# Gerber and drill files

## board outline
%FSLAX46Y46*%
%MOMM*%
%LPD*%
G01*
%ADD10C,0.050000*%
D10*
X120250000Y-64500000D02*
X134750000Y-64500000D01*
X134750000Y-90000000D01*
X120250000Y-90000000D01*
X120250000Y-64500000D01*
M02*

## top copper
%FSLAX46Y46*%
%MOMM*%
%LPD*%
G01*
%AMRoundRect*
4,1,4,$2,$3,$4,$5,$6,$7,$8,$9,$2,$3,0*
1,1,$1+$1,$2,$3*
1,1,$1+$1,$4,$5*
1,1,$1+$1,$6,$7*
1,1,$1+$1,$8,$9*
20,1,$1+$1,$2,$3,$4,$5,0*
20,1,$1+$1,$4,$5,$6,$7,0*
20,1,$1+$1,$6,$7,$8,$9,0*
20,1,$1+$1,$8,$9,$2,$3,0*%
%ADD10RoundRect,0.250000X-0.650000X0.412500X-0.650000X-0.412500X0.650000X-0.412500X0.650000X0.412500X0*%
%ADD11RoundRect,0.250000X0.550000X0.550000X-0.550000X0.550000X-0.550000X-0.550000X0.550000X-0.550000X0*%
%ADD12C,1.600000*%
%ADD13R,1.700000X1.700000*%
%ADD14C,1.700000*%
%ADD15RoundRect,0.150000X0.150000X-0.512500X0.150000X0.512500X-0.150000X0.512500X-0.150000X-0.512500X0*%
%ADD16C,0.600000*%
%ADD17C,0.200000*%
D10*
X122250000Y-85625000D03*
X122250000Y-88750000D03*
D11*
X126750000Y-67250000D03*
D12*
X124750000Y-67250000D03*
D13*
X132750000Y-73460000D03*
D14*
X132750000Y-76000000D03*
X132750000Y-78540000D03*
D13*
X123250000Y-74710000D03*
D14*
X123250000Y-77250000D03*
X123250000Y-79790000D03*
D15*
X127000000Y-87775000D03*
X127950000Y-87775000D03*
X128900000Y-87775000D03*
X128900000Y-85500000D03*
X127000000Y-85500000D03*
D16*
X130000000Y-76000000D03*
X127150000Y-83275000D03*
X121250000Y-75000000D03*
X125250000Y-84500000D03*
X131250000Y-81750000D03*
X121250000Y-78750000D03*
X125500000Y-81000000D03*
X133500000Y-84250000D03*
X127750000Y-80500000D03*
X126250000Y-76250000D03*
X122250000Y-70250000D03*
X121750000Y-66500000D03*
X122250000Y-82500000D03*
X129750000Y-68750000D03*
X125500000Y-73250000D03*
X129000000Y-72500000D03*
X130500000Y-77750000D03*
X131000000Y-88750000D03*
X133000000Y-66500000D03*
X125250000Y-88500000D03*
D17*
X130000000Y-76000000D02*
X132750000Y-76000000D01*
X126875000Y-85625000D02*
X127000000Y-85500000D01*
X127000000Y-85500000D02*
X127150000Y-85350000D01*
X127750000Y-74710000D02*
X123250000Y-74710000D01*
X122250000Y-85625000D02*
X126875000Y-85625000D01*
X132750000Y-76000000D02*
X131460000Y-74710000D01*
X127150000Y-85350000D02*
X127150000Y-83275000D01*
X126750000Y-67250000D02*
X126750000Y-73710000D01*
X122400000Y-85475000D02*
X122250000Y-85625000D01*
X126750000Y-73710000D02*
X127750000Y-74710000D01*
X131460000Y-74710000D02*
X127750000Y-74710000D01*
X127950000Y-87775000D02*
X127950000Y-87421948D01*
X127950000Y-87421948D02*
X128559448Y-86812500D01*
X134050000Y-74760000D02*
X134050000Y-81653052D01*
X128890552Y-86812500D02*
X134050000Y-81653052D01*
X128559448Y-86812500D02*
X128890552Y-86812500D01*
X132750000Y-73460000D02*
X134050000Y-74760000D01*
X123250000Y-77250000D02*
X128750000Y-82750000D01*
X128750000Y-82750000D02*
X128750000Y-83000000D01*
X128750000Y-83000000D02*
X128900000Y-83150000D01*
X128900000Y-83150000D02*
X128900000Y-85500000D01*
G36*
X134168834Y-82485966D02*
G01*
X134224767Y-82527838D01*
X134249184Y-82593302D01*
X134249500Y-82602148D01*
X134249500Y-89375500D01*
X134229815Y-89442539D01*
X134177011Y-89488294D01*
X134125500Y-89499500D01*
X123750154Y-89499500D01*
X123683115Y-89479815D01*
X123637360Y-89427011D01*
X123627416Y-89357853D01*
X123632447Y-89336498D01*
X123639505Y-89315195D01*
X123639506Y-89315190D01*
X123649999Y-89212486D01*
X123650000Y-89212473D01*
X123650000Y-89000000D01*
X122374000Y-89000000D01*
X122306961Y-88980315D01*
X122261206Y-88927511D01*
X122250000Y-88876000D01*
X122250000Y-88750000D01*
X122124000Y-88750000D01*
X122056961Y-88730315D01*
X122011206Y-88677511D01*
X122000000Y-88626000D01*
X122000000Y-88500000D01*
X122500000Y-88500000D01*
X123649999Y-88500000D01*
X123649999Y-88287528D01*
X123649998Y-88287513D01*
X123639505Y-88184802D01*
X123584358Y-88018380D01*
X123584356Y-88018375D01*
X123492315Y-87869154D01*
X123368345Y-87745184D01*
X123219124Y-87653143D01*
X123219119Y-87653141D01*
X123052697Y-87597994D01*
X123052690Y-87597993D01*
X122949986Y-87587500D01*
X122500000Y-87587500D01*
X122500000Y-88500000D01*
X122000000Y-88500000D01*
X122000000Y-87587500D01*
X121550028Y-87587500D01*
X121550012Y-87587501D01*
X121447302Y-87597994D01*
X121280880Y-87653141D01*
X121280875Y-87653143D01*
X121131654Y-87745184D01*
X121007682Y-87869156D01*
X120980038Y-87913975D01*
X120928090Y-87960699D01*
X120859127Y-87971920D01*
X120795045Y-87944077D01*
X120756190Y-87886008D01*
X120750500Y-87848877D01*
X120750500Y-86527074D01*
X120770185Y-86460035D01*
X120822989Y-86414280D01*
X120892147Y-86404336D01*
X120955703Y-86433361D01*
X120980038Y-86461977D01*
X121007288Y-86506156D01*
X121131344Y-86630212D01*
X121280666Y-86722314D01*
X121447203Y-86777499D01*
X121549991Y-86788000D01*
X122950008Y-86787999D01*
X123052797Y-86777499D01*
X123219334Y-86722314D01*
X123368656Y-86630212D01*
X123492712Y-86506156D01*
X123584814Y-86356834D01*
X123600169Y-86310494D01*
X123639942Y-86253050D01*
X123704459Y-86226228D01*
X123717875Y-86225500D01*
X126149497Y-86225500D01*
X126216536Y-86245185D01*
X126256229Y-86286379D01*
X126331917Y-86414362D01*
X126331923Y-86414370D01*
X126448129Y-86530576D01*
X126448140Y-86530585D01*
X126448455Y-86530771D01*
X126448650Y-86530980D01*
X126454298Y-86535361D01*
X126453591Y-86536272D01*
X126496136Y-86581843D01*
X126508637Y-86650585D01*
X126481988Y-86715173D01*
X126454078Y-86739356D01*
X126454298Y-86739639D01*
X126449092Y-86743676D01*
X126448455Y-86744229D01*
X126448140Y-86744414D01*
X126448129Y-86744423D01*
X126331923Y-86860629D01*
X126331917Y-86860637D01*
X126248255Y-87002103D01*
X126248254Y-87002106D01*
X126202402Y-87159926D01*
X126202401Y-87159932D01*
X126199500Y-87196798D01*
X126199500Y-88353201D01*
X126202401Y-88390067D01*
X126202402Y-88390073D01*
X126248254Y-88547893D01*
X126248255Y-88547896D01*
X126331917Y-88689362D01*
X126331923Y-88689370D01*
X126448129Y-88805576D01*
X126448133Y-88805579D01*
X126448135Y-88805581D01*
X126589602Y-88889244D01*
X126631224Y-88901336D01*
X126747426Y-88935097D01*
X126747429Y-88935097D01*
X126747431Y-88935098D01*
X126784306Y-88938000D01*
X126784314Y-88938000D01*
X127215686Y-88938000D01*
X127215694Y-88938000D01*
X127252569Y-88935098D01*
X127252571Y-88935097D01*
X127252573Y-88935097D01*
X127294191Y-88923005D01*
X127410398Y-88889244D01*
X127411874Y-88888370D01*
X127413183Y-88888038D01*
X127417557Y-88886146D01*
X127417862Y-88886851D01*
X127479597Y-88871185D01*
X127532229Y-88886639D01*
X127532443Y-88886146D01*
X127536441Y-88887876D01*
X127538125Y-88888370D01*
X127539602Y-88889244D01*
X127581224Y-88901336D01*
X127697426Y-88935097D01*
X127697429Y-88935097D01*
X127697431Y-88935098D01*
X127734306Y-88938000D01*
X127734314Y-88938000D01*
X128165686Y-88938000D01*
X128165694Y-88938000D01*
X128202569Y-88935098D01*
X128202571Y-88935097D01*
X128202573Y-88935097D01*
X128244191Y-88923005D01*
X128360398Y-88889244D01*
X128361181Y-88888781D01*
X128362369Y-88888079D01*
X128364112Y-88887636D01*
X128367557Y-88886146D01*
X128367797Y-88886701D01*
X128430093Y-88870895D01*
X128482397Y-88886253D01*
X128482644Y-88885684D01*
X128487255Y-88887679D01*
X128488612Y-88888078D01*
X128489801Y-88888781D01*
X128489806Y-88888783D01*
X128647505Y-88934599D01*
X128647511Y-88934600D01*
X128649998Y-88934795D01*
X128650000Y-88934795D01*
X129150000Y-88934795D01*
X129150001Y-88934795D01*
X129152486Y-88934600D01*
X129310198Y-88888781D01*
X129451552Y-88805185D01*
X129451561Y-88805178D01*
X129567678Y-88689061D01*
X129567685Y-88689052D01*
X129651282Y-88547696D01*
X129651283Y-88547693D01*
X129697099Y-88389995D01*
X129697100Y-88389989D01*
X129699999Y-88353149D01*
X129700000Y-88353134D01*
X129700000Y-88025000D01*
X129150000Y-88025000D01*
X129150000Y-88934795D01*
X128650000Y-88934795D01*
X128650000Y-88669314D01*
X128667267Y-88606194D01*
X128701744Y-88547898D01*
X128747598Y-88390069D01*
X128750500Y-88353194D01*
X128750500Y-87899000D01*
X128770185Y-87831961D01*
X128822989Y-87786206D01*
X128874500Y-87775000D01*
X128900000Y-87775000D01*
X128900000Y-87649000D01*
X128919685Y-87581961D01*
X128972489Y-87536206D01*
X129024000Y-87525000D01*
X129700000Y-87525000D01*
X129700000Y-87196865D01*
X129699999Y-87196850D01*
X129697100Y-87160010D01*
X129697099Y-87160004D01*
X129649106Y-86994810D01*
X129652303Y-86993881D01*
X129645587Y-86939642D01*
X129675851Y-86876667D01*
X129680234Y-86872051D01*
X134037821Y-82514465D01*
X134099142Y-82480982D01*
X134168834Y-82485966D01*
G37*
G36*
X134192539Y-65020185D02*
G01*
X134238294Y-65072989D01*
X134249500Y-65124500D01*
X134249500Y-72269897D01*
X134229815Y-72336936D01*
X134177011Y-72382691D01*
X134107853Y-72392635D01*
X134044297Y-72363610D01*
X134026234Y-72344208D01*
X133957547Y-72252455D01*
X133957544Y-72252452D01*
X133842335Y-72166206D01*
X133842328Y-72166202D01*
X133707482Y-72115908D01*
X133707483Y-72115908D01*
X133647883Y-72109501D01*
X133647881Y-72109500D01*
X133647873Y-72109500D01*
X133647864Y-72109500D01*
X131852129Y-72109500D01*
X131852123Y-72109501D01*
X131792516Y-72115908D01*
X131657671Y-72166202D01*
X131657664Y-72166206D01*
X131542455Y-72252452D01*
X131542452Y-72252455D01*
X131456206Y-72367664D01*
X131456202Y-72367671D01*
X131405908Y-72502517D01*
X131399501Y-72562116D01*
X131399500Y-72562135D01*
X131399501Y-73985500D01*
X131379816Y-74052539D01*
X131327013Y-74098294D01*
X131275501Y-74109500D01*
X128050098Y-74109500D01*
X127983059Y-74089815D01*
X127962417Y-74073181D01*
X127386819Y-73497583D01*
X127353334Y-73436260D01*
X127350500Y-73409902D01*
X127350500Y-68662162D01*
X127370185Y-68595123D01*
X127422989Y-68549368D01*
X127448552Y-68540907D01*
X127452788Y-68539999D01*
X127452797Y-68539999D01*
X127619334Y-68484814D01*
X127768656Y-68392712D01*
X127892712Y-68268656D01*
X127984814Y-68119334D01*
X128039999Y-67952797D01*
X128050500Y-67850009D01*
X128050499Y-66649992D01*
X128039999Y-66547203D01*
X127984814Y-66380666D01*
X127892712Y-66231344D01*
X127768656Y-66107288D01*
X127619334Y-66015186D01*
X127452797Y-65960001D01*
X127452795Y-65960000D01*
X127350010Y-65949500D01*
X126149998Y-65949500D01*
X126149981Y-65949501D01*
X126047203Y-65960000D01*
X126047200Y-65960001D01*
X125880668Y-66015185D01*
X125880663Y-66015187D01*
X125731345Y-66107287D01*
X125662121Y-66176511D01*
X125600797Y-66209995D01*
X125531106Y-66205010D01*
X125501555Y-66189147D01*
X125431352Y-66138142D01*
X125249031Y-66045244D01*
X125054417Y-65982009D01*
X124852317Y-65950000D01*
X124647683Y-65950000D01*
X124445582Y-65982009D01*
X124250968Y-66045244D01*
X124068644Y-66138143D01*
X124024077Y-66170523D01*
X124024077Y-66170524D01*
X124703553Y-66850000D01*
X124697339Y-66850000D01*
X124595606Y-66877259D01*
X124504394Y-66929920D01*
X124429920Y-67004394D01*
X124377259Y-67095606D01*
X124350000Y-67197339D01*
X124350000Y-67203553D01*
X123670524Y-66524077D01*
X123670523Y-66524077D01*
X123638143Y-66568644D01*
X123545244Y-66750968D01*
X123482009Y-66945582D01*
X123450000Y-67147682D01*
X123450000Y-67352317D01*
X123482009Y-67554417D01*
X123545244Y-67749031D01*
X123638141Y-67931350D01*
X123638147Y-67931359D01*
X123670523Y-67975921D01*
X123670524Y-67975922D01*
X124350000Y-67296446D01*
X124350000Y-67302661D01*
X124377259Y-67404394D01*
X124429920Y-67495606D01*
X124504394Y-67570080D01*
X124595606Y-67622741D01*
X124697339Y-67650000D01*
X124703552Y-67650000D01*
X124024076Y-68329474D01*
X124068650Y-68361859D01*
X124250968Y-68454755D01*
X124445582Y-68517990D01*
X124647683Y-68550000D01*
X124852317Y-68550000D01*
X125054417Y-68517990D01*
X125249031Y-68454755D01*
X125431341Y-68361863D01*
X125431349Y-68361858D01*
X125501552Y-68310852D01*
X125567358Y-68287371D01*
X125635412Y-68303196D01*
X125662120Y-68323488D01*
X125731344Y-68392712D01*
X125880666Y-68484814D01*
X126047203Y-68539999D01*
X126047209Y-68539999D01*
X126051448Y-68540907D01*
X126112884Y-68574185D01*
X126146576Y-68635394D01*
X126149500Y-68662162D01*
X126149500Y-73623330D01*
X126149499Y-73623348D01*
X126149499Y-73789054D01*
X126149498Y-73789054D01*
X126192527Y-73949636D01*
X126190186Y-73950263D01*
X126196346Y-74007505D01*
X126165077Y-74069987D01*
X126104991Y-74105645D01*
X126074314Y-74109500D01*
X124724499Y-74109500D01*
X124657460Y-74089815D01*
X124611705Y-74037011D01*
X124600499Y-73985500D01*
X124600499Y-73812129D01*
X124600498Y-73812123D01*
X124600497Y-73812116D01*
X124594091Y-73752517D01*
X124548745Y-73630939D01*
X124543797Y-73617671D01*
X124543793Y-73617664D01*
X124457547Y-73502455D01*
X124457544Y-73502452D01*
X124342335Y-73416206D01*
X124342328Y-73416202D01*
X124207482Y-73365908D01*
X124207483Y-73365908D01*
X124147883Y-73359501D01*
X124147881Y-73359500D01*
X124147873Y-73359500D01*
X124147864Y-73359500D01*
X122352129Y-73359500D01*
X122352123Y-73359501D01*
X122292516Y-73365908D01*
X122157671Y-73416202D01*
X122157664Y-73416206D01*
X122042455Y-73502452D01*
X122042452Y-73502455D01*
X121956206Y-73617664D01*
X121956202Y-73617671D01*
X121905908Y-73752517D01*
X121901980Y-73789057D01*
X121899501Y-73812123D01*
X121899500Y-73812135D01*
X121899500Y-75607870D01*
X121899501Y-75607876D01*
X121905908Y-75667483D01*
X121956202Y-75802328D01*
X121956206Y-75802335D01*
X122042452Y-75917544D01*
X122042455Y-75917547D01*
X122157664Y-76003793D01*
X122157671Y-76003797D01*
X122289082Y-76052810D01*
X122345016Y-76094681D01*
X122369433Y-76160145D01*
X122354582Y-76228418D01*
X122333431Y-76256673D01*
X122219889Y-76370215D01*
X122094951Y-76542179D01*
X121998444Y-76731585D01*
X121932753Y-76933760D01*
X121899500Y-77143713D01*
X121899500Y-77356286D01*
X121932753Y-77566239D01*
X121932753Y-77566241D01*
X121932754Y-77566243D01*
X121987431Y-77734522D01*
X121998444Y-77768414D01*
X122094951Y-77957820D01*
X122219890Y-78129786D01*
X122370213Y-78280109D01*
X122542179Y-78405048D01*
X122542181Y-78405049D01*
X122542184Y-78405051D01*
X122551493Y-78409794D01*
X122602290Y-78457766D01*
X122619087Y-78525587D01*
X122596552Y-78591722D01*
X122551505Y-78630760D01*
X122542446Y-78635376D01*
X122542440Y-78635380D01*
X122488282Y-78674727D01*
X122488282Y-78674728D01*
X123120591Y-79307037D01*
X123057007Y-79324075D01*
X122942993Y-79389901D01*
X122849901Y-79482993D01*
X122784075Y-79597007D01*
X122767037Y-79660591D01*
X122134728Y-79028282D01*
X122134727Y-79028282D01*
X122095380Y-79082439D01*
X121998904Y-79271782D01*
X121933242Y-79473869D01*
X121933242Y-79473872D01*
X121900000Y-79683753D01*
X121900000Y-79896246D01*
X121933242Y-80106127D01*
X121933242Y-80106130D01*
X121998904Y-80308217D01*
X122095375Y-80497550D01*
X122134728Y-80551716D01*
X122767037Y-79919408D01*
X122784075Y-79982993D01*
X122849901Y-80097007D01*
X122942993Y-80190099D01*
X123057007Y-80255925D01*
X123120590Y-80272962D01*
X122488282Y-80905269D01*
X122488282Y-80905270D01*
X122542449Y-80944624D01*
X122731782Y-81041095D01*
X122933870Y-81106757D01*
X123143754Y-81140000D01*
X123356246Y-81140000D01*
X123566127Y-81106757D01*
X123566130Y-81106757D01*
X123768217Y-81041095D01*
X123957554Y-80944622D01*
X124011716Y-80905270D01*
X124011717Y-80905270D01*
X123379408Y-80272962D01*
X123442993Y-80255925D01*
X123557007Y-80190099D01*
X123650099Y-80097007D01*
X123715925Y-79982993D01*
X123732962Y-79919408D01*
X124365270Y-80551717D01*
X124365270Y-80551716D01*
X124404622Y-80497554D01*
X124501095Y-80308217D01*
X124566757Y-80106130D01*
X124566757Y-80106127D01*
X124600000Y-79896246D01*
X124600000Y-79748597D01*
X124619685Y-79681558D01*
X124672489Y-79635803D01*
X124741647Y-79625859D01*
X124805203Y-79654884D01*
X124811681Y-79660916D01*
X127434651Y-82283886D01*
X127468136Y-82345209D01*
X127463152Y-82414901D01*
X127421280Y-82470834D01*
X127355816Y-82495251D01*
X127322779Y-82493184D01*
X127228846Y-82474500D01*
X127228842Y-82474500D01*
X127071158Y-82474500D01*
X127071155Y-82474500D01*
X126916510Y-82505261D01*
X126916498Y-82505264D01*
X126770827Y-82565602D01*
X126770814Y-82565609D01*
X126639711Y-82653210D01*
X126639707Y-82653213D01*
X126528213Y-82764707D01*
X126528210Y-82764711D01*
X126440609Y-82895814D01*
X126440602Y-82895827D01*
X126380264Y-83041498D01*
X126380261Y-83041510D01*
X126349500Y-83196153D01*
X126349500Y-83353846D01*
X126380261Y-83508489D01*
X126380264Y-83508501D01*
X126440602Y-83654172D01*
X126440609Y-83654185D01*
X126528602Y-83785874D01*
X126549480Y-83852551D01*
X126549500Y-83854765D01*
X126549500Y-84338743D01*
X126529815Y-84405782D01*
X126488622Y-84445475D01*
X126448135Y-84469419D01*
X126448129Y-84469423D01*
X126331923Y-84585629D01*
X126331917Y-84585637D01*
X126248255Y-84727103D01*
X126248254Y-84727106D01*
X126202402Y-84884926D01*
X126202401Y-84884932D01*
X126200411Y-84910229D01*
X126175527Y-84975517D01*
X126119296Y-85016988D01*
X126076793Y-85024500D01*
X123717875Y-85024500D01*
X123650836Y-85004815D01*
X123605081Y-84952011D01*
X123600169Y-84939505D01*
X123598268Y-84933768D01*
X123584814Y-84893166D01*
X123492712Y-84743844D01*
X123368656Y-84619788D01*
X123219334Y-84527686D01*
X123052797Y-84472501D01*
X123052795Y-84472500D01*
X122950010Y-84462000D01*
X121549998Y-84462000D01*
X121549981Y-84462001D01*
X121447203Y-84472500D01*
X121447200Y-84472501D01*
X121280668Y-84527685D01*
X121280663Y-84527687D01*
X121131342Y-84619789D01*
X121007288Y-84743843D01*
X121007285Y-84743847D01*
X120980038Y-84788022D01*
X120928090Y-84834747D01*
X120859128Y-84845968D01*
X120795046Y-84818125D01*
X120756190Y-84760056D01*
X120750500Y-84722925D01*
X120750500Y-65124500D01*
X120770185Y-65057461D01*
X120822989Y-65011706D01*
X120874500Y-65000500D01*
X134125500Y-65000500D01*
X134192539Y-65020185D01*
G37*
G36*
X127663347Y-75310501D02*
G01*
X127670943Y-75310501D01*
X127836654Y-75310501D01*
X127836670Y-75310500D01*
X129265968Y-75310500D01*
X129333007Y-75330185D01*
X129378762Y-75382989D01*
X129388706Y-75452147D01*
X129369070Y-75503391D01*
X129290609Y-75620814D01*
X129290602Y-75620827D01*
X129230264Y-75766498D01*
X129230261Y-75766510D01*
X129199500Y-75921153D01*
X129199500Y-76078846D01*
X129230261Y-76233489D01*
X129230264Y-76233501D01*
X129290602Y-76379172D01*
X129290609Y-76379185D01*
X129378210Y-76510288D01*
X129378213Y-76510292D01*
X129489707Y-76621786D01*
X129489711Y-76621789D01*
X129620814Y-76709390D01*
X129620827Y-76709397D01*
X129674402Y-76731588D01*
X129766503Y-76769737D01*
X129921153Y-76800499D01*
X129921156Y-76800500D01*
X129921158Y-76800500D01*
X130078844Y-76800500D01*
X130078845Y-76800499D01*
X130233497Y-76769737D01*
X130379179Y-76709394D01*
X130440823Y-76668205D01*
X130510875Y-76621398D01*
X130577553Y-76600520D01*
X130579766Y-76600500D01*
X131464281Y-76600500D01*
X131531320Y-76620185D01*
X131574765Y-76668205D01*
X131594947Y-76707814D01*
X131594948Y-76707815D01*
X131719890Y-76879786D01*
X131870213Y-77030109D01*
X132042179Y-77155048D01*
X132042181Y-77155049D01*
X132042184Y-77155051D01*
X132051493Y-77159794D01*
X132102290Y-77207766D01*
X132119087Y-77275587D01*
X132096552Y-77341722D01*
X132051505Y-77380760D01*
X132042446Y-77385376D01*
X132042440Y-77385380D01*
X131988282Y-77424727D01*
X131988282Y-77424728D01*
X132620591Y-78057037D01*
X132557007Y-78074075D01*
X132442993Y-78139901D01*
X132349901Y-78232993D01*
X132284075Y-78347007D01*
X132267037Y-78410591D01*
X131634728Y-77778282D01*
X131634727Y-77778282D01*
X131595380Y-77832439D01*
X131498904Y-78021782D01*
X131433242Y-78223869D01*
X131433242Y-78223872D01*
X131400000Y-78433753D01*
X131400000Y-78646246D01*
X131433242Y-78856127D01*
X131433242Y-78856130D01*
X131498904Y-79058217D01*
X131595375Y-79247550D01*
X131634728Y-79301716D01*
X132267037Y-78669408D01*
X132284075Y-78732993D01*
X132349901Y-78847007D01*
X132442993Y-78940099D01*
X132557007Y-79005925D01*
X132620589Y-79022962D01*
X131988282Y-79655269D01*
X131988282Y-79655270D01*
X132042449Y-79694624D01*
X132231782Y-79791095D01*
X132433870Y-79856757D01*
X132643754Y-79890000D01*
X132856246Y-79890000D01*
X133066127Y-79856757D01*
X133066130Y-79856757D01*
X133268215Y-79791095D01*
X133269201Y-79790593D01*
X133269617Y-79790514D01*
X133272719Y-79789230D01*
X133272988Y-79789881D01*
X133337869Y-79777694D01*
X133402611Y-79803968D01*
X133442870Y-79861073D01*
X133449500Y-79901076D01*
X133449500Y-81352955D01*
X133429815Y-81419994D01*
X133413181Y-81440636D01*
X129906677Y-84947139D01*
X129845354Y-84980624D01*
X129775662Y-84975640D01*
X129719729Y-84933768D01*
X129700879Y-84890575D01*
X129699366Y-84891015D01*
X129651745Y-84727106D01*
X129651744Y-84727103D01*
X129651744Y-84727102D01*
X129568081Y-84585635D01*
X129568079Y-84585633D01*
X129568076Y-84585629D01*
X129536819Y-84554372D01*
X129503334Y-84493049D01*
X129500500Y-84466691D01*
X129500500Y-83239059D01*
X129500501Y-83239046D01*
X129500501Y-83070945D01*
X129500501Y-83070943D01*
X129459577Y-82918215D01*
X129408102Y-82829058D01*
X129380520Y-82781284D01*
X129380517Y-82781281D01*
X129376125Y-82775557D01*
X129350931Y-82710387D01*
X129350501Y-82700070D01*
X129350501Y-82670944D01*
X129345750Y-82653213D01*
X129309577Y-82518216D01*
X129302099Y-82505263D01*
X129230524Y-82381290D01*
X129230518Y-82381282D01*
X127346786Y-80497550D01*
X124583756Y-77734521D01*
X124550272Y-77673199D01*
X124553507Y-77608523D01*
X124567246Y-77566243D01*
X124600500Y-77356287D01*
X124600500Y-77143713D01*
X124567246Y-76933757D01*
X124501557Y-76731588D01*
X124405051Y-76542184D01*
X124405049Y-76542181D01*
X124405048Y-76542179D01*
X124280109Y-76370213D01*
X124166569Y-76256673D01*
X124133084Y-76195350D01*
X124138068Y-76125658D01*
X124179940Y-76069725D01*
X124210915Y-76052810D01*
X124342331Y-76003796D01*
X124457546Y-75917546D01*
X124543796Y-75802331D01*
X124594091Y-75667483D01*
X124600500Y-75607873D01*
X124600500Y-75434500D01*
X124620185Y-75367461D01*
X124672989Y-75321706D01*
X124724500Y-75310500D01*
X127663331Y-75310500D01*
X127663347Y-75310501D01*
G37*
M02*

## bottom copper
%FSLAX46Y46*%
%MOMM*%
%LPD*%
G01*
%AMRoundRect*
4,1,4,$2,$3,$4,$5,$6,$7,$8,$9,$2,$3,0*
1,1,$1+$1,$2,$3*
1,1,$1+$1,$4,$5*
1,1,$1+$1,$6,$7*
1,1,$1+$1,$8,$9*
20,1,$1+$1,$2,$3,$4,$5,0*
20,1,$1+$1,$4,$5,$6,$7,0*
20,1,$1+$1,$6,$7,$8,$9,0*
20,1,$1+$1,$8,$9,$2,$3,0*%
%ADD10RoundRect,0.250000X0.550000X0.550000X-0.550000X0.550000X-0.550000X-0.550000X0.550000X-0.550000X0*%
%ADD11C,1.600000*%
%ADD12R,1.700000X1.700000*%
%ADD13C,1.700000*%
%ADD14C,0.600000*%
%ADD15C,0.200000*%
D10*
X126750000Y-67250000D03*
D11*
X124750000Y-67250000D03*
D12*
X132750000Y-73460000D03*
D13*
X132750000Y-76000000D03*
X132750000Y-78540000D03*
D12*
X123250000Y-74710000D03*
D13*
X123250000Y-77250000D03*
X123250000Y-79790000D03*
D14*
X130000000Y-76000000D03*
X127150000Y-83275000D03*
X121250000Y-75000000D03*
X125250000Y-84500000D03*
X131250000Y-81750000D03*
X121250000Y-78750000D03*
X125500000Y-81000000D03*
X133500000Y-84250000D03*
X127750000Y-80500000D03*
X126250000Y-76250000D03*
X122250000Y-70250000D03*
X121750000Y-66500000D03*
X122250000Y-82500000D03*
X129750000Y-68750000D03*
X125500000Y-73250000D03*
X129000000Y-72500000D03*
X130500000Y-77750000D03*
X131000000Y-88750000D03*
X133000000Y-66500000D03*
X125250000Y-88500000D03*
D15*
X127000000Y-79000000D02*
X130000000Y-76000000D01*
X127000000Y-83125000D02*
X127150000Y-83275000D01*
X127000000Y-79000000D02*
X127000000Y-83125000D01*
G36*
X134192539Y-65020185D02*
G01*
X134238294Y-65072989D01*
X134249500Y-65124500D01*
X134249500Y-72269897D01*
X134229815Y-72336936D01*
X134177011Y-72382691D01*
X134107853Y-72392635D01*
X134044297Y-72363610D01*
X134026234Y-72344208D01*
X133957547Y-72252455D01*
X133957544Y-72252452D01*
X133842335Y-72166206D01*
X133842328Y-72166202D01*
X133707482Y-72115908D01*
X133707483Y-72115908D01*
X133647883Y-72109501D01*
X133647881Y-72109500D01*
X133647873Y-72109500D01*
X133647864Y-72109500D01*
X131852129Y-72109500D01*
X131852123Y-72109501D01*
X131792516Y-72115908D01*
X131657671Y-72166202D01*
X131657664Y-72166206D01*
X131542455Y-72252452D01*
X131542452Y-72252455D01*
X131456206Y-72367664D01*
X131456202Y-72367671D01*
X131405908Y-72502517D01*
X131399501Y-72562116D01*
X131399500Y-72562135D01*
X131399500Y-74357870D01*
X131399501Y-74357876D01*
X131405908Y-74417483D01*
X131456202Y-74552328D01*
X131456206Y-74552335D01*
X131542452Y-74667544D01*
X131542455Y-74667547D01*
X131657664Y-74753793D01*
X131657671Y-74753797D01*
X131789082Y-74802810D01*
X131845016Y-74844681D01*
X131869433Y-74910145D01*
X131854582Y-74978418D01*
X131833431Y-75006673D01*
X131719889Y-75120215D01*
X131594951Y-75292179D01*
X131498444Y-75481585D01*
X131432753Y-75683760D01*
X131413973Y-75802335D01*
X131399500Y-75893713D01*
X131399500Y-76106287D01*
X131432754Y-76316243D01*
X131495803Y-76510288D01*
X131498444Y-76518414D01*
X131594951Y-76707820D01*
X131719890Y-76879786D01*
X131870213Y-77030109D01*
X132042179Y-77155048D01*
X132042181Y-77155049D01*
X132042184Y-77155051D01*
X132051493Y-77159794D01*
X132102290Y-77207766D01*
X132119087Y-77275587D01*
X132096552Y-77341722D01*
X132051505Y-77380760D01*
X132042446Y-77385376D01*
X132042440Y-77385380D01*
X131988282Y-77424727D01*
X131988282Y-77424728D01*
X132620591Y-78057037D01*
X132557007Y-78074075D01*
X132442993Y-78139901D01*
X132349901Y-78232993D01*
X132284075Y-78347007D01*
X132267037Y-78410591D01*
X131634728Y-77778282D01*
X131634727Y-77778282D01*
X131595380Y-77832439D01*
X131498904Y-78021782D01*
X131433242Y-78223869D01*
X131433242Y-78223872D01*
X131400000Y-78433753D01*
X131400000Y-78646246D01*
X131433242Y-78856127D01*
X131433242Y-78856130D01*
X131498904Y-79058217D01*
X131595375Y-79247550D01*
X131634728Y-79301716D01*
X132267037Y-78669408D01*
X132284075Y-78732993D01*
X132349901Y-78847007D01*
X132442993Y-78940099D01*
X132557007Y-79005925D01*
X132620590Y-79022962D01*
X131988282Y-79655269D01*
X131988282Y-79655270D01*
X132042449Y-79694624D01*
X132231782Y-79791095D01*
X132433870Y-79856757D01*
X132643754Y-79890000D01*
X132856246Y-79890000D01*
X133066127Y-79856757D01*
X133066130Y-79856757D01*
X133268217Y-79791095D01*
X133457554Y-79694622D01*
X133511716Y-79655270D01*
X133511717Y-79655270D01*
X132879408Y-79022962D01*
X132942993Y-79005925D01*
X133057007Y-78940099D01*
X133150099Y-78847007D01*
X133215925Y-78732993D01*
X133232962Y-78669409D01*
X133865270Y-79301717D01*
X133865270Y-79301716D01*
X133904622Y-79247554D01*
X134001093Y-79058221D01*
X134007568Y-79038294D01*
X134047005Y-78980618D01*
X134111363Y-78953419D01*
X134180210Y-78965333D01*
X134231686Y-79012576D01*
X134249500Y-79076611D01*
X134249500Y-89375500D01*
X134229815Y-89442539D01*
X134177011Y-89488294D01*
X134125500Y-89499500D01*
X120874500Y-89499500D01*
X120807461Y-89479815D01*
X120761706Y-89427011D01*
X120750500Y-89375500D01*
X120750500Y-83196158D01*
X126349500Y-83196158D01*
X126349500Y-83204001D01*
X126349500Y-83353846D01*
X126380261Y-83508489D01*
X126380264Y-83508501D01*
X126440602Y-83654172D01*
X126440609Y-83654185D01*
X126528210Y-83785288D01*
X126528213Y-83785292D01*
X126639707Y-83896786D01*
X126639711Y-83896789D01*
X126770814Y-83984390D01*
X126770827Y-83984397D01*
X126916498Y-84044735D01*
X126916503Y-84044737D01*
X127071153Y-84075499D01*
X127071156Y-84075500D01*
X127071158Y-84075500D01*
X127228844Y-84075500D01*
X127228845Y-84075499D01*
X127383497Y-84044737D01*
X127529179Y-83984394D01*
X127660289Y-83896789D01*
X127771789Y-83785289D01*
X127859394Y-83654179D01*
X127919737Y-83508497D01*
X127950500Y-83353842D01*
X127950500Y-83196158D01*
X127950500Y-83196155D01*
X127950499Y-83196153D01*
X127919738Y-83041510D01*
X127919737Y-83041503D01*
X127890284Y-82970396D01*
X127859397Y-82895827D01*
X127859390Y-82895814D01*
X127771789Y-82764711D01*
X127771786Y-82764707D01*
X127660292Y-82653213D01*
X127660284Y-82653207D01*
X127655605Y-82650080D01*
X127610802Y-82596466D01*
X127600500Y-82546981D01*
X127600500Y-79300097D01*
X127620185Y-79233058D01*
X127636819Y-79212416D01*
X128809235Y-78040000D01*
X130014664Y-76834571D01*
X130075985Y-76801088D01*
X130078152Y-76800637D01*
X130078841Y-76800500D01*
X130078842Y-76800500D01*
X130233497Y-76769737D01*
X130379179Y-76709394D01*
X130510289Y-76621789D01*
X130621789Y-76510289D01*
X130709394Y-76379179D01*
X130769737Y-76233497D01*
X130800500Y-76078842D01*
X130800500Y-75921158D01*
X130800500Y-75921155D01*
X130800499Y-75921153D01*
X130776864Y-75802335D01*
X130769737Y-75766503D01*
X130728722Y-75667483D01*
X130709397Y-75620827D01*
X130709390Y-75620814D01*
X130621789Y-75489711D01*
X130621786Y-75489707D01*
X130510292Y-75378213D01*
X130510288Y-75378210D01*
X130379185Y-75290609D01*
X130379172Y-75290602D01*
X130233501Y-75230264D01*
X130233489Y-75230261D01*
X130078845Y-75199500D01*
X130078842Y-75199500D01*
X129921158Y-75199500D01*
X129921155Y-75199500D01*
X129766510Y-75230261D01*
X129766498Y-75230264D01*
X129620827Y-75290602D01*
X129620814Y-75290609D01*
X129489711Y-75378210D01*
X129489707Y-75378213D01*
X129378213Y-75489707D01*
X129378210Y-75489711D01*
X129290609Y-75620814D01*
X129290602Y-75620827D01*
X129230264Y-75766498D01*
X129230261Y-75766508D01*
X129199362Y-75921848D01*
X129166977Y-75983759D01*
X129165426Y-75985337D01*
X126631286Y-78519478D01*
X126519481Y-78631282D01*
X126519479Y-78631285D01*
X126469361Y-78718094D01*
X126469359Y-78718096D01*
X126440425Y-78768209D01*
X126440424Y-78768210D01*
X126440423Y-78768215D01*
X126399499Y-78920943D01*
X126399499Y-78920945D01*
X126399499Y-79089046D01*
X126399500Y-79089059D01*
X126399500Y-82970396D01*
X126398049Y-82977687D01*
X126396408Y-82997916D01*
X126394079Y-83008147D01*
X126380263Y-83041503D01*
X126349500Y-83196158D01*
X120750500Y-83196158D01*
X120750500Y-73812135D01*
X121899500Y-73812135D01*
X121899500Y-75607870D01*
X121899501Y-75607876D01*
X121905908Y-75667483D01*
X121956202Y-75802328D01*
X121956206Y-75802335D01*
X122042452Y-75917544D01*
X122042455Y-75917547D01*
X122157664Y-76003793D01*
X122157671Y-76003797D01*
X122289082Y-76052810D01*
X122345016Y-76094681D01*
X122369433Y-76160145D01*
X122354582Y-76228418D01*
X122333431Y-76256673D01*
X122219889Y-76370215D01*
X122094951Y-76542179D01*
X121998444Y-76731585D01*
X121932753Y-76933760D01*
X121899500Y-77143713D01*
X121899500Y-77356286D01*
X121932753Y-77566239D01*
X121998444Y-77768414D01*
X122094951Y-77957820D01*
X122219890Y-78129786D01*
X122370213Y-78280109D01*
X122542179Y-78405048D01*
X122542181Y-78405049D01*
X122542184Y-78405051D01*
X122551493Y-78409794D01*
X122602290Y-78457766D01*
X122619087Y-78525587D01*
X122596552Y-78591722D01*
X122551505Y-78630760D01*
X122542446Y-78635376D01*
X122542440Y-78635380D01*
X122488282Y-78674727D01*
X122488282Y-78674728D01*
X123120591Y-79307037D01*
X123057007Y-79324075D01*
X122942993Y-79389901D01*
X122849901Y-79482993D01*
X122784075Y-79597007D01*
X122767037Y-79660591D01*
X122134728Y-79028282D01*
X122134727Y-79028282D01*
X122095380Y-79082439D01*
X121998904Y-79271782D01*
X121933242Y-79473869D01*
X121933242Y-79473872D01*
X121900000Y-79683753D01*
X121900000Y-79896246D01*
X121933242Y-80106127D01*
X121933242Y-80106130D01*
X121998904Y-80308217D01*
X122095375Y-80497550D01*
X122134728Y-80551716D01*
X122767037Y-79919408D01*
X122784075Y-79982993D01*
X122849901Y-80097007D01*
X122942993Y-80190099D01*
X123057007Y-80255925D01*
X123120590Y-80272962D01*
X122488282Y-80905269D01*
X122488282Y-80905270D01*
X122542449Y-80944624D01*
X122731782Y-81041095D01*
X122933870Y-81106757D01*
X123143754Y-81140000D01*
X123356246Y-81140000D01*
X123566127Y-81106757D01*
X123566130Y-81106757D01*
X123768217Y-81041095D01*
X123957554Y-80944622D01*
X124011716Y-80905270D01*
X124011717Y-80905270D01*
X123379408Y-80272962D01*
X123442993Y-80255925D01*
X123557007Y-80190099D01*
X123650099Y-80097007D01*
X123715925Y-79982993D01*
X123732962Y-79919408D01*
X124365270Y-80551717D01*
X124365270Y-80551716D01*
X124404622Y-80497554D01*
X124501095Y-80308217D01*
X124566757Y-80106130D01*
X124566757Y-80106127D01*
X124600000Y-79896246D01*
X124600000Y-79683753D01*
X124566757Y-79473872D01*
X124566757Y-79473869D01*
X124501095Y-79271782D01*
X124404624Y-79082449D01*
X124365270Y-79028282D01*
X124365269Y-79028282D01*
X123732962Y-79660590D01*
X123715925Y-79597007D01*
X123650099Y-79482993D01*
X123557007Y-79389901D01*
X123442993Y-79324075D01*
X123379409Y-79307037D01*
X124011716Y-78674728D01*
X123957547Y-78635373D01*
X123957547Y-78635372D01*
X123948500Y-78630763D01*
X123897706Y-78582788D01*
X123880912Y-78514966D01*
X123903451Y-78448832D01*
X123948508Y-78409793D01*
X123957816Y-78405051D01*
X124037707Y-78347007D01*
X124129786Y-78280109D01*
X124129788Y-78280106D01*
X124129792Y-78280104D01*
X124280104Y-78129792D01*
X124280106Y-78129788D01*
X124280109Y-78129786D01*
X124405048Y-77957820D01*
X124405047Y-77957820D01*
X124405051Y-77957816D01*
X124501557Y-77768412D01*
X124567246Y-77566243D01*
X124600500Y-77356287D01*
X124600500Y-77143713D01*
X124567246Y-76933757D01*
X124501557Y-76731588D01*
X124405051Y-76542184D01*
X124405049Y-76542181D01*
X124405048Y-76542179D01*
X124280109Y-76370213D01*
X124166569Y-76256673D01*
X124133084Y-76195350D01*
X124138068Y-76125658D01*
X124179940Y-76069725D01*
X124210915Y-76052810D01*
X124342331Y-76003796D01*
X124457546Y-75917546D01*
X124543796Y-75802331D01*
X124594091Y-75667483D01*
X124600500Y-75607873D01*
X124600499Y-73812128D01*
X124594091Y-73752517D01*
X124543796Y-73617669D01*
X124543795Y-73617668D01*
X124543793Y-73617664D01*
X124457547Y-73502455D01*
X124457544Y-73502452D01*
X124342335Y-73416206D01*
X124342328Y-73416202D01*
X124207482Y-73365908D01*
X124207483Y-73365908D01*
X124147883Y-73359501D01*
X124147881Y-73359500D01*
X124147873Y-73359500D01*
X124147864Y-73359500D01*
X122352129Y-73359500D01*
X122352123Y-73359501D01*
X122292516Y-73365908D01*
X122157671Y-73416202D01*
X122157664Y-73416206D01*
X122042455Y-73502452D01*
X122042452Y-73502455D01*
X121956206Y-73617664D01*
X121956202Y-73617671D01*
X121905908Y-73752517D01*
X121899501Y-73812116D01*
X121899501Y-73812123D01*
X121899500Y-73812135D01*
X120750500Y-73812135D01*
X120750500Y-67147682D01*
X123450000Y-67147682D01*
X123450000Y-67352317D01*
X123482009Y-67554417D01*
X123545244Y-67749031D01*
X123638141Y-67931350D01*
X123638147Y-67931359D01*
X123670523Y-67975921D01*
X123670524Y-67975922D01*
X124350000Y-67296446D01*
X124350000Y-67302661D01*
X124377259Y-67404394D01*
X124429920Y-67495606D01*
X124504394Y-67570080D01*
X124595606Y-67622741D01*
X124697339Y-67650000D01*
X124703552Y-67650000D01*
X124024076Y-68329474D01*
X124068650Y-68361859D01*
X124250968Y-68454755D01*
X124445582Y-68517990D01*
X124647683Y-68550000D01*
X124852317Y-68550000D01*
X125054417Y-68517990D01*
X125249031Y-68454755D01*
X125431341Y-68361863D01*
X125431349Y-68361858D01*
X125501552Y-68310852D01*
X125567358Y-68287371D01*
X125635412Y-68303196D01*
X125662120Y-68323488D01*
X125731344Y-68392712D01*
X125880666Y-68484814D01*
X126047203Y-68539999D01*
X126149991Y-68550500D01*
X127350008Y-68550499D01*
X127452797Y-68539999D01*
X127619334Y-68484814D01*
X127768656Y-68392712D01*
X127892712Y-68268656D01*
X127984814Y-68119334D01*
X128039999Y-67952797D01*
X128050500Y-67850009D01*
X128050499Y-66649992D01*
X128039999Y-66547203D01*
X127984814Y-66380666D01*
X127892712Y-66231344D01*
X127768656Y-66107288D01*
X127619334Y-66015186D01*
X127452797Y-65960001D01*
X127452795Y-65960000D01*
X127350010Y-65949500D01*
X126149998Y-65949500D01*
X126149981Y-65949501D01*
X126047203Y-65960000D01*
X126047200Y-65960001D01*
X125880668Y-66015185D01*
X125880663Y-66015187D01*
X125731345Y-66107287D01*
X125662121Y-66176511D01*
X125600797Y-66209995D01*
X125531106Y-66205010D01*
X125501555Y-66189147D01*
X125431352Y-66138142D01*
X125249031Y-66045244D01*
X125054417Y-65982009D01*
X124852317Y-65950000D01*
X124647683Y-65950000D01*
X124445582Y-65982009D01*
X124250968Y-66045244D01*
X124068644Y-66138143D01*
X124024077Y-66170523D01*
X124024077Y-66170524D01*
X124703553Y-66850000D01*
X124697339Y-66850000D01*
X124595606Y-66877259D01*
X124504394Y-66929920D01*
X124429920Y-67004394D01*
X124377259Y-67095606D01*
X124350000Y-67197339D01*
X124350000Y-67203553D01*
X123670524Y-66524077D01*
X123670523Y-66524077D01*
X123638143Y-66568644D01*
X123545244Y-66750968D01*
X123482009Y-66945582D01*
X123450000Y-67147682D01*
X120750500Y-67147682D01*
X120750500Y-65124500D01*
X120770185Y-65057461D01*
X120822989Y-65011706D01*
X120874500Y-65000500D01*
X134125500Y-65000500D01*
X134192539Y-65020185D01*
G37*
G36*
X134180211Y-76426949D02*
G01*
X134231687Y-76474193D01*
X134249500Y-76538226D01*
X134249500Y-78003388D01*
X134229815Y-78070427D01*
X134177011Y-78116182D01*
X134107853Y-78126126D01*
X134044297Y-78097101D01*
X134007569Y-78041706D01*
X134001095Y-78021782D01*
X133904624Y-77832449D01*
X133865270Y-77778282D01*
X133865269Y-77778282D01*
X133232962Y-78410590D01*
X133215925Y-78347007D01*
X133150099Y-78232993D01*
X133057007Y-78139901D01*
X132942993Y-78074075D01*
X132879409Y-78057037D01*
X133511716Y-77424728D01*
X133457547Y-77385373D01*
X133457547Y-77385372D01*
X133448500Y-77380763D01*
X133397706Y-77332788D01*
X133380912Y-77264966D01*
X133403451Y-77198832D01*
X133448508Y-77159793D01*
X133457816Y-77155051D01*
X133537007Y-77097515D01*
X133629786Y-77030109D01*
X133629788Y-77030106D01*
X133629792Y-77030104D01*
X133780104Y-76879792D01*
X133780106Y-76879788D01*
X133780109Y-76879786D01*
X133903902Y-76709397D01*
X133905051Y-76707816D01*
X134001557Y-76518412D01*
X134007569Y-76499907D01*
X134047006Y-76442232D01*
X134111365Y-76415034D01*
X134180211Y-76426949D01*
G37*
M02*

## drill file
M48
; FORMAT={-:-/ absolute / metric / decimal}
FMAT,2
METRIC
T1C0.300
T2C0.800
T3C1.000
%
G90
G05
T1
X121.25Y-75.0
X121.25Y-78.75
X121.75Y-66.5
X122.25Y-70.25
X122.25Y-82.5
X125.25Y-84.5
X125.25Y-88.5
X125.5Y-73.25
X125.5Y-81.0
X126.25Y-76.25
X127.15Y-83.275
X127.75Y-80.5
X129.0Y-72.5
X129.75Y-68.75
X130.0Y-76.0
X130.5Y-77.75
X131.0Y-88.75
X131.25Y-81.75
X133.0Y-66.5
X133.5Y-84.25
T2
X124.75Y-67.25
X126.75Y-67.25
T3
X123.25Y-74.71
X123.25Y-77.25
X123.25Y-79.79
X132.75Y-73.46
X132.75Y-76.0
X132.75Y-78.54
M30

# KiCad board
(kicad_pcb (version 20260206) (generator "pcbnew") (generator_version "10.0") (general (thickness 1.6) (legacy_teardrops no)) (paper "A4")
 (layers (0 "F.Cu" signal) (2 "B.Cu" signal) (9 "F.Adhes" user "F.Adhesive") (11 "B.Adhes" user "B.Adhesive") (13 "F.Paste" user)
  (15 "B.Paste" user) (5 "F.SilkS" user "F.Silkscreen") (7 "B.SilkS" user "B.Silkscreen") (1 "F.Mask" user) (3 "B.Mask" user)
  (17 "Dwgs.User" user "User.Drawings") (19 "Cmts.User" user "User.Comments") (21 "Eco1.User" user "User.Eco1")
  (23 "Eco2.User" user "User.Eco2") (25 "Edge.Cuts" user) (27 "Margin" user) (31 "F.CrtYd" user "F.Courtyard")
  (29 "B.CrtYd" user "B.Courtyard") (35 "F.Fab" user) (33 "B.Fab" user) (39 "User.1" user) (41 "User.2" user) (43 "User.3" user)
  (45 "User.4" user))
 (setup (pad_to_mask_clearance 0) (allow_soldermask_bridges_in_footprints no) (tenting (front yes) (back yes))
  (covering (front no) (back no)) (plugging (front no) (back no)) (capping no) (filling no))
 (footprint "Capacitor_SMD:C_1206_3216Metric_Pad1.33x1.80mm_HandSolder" (layer "F.Cu") (at 122.25 87.1875 -90)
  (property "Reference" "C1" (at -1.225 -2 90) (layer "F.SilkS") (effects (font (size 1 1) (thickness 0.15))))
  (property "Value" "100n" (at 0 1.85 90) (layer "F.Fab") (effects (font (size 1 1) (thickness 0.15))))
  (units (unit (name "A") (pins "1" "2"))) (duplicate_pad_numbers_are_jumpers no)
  (pad "1" smd roundrect (at -1.5625 0 270) (size 1.325 1.8) (layers "F.Cu" "F.Mask" "F.Paste") (roundrect_rratio 0.188679) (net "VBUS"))
  (pad "2" smd roundrect (at 1.5625 0 270) (size 1.325 1.8) (layers "F.Cu" "F.Mask" "F.Paste") (roundrect_rratio 0.188679) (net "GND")))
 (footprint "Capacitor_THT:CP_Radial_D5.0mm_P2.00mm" (layer "F.Cu") (at 126.75 67.25 180)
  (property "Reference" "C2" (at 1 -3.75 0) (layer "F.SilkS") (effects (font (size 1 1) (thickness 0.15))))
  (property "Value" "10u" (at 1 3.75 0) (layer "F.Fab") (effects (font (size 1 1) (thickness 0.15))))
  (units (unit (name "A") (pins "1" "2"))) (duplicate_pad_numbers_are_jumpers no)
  (pad "1" thru_hole roundrect (at 0 0 180) (size 1.6 1.6) (drill 0.8) (layers "*.Cu" "*.Mask") (remove_unused_layers no)
   (roundrect_rratio 0.15625) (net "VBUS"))
  (pad "2" thru_hole circle (at 2 0 180) (size 1.6 1.6) (drill 0.8) (layers "*.Cu" "*.Mask") (remove_unused_layers no) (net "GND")))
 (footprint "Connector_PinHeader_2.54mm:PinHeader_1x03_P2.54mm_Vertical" (layer "F.Cu") (at 132.75 73.46)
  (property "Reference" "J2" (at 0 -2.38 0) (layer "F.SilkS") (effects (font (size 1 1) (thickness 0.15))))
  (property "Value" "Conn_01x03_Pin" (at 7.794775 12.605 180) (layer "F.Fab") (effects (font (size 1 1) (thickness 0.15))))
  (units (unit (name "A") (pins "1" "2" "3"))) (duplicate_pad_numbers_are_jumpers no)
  (pad "1" thru_hole rect (at 0 0) (size 1.7 1.7) (drill 1) (layers "*.Cu" "*.Mask") (remove_unused_layers no) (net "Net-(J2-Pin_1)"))
  (pad "2" thru_hole circle (at 0 2.54) (size 1.7 1.7) (drill 1) (layers "*.Cu" "*.Mask") (remove_unused_layers no) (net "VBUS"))
  (pad "3" thru_hole circle (at 0 5.08) (size 1.7 1.7) (drill 1) (layers "*.Cu" "*.Mask") (remove_unused_layers no) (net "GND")))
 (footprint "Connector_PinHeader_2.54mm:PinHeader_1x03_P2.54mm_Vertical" (layer "F.Cu") (at 123.25 74.71)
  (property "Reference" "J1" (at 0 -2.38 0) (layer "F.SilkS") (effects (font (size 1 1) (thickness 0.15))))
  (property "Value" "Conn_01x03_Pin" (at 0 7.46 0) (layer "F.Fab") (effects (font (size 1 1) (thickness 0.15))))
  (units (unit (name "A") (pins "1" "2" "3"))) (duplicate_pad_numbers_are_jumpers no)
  (pad "1" thru_hole rect (at 0 0) (size 1.7 1.7) (drill 1) (layers "*.Cu" "*.Mask") (remove_unused_layers no) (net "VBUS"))
  (pad "2" thru_hole circle (at 0 2.54) (size 1.7 1.7) (drill 1) (layers "*.Cu" "*.Mask") (remove_unused_layers no) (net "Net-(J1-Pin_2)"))
  (pad "3" thru_hole circle (at 0 5.08) (size 1.7 1.7) (drill 1) (layers "*.Cu" "*.Mask") (remove_unused_layers no) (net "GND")))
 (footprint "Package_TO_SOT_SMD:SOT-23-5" (layer "F.Cu") (at 127.95 86.6375 90)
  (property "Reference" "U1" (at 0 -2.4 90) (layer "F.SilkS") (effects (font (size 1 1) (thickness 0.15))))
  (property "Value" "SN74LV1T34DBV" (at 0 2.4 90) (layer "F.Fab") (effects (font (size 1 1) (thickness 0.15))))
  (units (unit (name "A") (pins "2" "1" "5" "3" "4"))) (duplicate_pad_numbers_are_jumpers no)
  (pad "1" smd roundrect (at -1.1375 -0.95 90) (size 1.325 0.6) (layers "F.Cu" "F.Mask" "F.Paste") (roundrect_rratio 0.25)
   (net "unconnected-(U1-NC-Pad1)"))
  (pad "2" smd roundrect (at -1.1375 0 90) (size 1.325 0.6) (layers "F.Cu" "F.Mask" "F.Paste") (roundrect_rratio 0.25)
   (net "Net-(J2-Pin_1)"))
  (pad "3" smd roundrect (at -1.1375 0.95 90) (size 1.325 0.6) (layers "F.Cu" "F.Mask" "F.Paste") (roundrect_rratio 0.25) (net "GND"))
  (pad "4" smd roundrect (at 1.1375 0.95 90) (size 1.325 0.6) (layers "F.Cu" "F.Mask" "F.Paste") (roundrect_rratio 0.25)
   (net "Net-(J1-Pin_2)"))
  (pad "5" smd roundrect (at 1.1375 -0.95 90) (size 1.325 0.6) (layers "F.Cu" "F.Mask" "F.Paste") (roundrect_rratio 0.25) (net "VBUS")))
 (gr_rect (start 120.25 64.5) (end 134.75 90) (stroke (width 0.05) (type default)) (fill no) (layer "Edge.Cuts"))
 (segment (start 130 76) (end 132.75 76) (width 0.2) (layer "F.Cu") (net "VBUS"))
 (segment (start 126.875 85.625) (end 127 85.5) (width 0.2) (layer "F.Cu") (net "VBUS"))
 (segment (start 127 85.5) (end 127.15 85.35) (width 0.2) (layer "F.Cu") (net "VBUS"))
 (segment (start 127.75 74.71) (end 123.25 74.71) (width 0.2) (layer "F.Cu") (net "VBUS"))
 (segment (start 122.25 85.625) (end 126.875 85.625) (width 0.2) (layer "F.Cu") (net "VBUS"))
 (segment (start 132.75 76) (end 131.46 74.71) (width 0.2) (layer "F.Cu") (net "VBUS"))
 (segment (start 127.15 85.35) (end 127.15 83.275) (width 0.2) (layer "F.Cu") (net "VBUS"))
 (segment (start 126.75 67.25) (end 126.75 73.71) (width 0.2) (layer "F.Cu") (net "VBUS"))
 (segment (start 122.4 85.475) (end 122.25 85.625) (width 0.2) (layer "F.Cu") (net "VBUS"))
 (segment (start 126.75 73.71) (end 127.75 74.71) (width 0.2) (layer "F.Cu") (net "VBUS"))
 (segment (start 131.46 74.71) (end 127.75 74.71) (width 0.2) (layer "F.Cu") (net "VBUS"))
 (via (at 130 76) (size 0.6) (drill 0.3) (layers "F.Cu" "B.Cu") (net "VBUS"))
 (via (at 127.15 83.275) (size 0.6) (drill 0.3) (layers "F.Cu" "B.Cu") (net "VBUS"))
 (segment (start 127 79) (end 130 76) (width 0.2) (layer "B.Cu") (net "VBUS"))
 (segment (start 127 83.125) (end 127.15 83.275) (width 0.2) (layer "B.Cu") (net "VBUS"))
 (segment (start 127 79) (end 127 83.125) (width 0.2) (layer "B.Cu") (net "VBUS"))
 (via (at 121.25 75) (size 0.6) (drill 0.3) (layers "F.Cu" "B.Cu") (free yes) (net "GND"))
 (via (at 125.25 84.5) (size 0.6) (drill 0.3) (layers "F.Cu" "B.Cu") (free yes) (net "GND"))
 (via (at 131.25 81.75) (size 0.6) (drill 0.3) (layers "F.Cu" "B.Cu") (free yes) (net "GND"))
 (via (at 121.25 78.75) (size 0.6) (drill 0.3) (layers "F.Cu" "B.Cu") (free yes) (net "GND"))
 (via (at 125.5 81) (size 0.6) (drill 0.3) (layers "F.Cu" "B.Cu") (free yes) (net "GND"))
 (via (at 133.5 84.25) (size 0.6) (drill 0.3) (layers "F.Cu" "B.Cu") (free yes) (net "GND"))
 (via (at 127.75 80.5) (size 0.6) (drill 0.3) (layers "F.Cu" "B.Cu") (free yes) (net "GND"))
 (via (at 126.25 76.25) (size 0.6) (drill 0.3) (layers "F.Cu" "B.Cu") (free yes) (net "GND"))
 (via (at 122.25 70.25) (size 0.6) (drill 0.3) (layers "F.Cu" "B.Cu") (free yes) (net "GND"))
 (via (at 121.75 66.5) (size 0.6) (drill 0.3) (layers "F.Cu" "B.Cu") (free yes) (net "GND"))
 (via (at 122.25 82.5) (size 0.6) (drill 0.3) (layers "F.Cu" "B.Cu") (free yes) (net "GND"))
 (via (at 129.75 68.75) (size 0.6) (drill 0.3) (layers "F.Cu" "B.Cu") (free yes) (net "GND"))
 (via (at 125.5 73.25) (size 0.6) (drill 0.3) (layers "F.Cu" "B.Cu") (free yes) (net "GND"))
 (via (at 129 72.5) (size 0.6) (drill 0.3) (layers "F.Cu" "B.Cu") (free yes) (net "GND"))
 (via (at 130.5 77.75) (size 0.6) (drill 0.3) (layers "F.Cu" "B.Cu") (free yes) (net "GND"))
 (via (at 131 88.75) (size 0.6) (drill 0.3) (layers "F.Cu" "B.Cu") (free yes) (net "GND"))
 (via (at 133 66.5) (size 0.6) (drill 0.3) (layers "F.Cu" "B.Cu") (free yes) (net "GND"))
 (via (at 125.25 88.5) (size 0.6) (drill 0.3) (layers "F.Cu" "B.Cu") (free yes) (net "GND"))
 (segment (start 127.95 87.775) (end 127.95 87.421948) (width 0.2) (layer "F.Cu") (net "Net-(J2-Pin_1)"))
 (segment (start 127.95 87.421948) (end 128.559448 86.8125) (width 0.2) (layer "F.Cu") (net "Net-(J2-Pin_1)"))
 (segment (start 134.05 74.76) (end 134.05 81.653052) (width 0.2) (layer "F.Cu") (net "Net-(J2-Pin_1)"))
 (segment (start 128.890552 86.8125) (end 134.05 81.653052) (width 0.2) (layer "F.Cu") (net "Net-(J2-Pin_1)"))
 (segment (start 128.559448 86.8125) (end 128.890552 86.8125) (width 0.2) (layer "F.Cu") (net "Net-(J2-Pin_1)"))
 (segment (start 132.75 73.46) (end 134.05 74.76) (width 0.2) (layer "F.Cu") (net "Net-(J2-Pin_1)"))
 (segment (start 123.25 77.25) (end 128.75 82.75) (width 0.2) (layer "F.Cu") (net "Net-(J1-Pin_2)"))
 (segment (start 128.75 82.75) (end 128.75 83) (width 0.2) (layer "F.Cu") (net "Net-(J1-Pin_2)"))
 (segment (start 128.75 83) (end 128.9 83.15) (width 0.2) (layer "F.Cu") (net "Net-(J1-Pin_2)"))
 (segment (start 128.9 83.15) (end 128.9 85.5) (width 0.2) (layer "F.Cu") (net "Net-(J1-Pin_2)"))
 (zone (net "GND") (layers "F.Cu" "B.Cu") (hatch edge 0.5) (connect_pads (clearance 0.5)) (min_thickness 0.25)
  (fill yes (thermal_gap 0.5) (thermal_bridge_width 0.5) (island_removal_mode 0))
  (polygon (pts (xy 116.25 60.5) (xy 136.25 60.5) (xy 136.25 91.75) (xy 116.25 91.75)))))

